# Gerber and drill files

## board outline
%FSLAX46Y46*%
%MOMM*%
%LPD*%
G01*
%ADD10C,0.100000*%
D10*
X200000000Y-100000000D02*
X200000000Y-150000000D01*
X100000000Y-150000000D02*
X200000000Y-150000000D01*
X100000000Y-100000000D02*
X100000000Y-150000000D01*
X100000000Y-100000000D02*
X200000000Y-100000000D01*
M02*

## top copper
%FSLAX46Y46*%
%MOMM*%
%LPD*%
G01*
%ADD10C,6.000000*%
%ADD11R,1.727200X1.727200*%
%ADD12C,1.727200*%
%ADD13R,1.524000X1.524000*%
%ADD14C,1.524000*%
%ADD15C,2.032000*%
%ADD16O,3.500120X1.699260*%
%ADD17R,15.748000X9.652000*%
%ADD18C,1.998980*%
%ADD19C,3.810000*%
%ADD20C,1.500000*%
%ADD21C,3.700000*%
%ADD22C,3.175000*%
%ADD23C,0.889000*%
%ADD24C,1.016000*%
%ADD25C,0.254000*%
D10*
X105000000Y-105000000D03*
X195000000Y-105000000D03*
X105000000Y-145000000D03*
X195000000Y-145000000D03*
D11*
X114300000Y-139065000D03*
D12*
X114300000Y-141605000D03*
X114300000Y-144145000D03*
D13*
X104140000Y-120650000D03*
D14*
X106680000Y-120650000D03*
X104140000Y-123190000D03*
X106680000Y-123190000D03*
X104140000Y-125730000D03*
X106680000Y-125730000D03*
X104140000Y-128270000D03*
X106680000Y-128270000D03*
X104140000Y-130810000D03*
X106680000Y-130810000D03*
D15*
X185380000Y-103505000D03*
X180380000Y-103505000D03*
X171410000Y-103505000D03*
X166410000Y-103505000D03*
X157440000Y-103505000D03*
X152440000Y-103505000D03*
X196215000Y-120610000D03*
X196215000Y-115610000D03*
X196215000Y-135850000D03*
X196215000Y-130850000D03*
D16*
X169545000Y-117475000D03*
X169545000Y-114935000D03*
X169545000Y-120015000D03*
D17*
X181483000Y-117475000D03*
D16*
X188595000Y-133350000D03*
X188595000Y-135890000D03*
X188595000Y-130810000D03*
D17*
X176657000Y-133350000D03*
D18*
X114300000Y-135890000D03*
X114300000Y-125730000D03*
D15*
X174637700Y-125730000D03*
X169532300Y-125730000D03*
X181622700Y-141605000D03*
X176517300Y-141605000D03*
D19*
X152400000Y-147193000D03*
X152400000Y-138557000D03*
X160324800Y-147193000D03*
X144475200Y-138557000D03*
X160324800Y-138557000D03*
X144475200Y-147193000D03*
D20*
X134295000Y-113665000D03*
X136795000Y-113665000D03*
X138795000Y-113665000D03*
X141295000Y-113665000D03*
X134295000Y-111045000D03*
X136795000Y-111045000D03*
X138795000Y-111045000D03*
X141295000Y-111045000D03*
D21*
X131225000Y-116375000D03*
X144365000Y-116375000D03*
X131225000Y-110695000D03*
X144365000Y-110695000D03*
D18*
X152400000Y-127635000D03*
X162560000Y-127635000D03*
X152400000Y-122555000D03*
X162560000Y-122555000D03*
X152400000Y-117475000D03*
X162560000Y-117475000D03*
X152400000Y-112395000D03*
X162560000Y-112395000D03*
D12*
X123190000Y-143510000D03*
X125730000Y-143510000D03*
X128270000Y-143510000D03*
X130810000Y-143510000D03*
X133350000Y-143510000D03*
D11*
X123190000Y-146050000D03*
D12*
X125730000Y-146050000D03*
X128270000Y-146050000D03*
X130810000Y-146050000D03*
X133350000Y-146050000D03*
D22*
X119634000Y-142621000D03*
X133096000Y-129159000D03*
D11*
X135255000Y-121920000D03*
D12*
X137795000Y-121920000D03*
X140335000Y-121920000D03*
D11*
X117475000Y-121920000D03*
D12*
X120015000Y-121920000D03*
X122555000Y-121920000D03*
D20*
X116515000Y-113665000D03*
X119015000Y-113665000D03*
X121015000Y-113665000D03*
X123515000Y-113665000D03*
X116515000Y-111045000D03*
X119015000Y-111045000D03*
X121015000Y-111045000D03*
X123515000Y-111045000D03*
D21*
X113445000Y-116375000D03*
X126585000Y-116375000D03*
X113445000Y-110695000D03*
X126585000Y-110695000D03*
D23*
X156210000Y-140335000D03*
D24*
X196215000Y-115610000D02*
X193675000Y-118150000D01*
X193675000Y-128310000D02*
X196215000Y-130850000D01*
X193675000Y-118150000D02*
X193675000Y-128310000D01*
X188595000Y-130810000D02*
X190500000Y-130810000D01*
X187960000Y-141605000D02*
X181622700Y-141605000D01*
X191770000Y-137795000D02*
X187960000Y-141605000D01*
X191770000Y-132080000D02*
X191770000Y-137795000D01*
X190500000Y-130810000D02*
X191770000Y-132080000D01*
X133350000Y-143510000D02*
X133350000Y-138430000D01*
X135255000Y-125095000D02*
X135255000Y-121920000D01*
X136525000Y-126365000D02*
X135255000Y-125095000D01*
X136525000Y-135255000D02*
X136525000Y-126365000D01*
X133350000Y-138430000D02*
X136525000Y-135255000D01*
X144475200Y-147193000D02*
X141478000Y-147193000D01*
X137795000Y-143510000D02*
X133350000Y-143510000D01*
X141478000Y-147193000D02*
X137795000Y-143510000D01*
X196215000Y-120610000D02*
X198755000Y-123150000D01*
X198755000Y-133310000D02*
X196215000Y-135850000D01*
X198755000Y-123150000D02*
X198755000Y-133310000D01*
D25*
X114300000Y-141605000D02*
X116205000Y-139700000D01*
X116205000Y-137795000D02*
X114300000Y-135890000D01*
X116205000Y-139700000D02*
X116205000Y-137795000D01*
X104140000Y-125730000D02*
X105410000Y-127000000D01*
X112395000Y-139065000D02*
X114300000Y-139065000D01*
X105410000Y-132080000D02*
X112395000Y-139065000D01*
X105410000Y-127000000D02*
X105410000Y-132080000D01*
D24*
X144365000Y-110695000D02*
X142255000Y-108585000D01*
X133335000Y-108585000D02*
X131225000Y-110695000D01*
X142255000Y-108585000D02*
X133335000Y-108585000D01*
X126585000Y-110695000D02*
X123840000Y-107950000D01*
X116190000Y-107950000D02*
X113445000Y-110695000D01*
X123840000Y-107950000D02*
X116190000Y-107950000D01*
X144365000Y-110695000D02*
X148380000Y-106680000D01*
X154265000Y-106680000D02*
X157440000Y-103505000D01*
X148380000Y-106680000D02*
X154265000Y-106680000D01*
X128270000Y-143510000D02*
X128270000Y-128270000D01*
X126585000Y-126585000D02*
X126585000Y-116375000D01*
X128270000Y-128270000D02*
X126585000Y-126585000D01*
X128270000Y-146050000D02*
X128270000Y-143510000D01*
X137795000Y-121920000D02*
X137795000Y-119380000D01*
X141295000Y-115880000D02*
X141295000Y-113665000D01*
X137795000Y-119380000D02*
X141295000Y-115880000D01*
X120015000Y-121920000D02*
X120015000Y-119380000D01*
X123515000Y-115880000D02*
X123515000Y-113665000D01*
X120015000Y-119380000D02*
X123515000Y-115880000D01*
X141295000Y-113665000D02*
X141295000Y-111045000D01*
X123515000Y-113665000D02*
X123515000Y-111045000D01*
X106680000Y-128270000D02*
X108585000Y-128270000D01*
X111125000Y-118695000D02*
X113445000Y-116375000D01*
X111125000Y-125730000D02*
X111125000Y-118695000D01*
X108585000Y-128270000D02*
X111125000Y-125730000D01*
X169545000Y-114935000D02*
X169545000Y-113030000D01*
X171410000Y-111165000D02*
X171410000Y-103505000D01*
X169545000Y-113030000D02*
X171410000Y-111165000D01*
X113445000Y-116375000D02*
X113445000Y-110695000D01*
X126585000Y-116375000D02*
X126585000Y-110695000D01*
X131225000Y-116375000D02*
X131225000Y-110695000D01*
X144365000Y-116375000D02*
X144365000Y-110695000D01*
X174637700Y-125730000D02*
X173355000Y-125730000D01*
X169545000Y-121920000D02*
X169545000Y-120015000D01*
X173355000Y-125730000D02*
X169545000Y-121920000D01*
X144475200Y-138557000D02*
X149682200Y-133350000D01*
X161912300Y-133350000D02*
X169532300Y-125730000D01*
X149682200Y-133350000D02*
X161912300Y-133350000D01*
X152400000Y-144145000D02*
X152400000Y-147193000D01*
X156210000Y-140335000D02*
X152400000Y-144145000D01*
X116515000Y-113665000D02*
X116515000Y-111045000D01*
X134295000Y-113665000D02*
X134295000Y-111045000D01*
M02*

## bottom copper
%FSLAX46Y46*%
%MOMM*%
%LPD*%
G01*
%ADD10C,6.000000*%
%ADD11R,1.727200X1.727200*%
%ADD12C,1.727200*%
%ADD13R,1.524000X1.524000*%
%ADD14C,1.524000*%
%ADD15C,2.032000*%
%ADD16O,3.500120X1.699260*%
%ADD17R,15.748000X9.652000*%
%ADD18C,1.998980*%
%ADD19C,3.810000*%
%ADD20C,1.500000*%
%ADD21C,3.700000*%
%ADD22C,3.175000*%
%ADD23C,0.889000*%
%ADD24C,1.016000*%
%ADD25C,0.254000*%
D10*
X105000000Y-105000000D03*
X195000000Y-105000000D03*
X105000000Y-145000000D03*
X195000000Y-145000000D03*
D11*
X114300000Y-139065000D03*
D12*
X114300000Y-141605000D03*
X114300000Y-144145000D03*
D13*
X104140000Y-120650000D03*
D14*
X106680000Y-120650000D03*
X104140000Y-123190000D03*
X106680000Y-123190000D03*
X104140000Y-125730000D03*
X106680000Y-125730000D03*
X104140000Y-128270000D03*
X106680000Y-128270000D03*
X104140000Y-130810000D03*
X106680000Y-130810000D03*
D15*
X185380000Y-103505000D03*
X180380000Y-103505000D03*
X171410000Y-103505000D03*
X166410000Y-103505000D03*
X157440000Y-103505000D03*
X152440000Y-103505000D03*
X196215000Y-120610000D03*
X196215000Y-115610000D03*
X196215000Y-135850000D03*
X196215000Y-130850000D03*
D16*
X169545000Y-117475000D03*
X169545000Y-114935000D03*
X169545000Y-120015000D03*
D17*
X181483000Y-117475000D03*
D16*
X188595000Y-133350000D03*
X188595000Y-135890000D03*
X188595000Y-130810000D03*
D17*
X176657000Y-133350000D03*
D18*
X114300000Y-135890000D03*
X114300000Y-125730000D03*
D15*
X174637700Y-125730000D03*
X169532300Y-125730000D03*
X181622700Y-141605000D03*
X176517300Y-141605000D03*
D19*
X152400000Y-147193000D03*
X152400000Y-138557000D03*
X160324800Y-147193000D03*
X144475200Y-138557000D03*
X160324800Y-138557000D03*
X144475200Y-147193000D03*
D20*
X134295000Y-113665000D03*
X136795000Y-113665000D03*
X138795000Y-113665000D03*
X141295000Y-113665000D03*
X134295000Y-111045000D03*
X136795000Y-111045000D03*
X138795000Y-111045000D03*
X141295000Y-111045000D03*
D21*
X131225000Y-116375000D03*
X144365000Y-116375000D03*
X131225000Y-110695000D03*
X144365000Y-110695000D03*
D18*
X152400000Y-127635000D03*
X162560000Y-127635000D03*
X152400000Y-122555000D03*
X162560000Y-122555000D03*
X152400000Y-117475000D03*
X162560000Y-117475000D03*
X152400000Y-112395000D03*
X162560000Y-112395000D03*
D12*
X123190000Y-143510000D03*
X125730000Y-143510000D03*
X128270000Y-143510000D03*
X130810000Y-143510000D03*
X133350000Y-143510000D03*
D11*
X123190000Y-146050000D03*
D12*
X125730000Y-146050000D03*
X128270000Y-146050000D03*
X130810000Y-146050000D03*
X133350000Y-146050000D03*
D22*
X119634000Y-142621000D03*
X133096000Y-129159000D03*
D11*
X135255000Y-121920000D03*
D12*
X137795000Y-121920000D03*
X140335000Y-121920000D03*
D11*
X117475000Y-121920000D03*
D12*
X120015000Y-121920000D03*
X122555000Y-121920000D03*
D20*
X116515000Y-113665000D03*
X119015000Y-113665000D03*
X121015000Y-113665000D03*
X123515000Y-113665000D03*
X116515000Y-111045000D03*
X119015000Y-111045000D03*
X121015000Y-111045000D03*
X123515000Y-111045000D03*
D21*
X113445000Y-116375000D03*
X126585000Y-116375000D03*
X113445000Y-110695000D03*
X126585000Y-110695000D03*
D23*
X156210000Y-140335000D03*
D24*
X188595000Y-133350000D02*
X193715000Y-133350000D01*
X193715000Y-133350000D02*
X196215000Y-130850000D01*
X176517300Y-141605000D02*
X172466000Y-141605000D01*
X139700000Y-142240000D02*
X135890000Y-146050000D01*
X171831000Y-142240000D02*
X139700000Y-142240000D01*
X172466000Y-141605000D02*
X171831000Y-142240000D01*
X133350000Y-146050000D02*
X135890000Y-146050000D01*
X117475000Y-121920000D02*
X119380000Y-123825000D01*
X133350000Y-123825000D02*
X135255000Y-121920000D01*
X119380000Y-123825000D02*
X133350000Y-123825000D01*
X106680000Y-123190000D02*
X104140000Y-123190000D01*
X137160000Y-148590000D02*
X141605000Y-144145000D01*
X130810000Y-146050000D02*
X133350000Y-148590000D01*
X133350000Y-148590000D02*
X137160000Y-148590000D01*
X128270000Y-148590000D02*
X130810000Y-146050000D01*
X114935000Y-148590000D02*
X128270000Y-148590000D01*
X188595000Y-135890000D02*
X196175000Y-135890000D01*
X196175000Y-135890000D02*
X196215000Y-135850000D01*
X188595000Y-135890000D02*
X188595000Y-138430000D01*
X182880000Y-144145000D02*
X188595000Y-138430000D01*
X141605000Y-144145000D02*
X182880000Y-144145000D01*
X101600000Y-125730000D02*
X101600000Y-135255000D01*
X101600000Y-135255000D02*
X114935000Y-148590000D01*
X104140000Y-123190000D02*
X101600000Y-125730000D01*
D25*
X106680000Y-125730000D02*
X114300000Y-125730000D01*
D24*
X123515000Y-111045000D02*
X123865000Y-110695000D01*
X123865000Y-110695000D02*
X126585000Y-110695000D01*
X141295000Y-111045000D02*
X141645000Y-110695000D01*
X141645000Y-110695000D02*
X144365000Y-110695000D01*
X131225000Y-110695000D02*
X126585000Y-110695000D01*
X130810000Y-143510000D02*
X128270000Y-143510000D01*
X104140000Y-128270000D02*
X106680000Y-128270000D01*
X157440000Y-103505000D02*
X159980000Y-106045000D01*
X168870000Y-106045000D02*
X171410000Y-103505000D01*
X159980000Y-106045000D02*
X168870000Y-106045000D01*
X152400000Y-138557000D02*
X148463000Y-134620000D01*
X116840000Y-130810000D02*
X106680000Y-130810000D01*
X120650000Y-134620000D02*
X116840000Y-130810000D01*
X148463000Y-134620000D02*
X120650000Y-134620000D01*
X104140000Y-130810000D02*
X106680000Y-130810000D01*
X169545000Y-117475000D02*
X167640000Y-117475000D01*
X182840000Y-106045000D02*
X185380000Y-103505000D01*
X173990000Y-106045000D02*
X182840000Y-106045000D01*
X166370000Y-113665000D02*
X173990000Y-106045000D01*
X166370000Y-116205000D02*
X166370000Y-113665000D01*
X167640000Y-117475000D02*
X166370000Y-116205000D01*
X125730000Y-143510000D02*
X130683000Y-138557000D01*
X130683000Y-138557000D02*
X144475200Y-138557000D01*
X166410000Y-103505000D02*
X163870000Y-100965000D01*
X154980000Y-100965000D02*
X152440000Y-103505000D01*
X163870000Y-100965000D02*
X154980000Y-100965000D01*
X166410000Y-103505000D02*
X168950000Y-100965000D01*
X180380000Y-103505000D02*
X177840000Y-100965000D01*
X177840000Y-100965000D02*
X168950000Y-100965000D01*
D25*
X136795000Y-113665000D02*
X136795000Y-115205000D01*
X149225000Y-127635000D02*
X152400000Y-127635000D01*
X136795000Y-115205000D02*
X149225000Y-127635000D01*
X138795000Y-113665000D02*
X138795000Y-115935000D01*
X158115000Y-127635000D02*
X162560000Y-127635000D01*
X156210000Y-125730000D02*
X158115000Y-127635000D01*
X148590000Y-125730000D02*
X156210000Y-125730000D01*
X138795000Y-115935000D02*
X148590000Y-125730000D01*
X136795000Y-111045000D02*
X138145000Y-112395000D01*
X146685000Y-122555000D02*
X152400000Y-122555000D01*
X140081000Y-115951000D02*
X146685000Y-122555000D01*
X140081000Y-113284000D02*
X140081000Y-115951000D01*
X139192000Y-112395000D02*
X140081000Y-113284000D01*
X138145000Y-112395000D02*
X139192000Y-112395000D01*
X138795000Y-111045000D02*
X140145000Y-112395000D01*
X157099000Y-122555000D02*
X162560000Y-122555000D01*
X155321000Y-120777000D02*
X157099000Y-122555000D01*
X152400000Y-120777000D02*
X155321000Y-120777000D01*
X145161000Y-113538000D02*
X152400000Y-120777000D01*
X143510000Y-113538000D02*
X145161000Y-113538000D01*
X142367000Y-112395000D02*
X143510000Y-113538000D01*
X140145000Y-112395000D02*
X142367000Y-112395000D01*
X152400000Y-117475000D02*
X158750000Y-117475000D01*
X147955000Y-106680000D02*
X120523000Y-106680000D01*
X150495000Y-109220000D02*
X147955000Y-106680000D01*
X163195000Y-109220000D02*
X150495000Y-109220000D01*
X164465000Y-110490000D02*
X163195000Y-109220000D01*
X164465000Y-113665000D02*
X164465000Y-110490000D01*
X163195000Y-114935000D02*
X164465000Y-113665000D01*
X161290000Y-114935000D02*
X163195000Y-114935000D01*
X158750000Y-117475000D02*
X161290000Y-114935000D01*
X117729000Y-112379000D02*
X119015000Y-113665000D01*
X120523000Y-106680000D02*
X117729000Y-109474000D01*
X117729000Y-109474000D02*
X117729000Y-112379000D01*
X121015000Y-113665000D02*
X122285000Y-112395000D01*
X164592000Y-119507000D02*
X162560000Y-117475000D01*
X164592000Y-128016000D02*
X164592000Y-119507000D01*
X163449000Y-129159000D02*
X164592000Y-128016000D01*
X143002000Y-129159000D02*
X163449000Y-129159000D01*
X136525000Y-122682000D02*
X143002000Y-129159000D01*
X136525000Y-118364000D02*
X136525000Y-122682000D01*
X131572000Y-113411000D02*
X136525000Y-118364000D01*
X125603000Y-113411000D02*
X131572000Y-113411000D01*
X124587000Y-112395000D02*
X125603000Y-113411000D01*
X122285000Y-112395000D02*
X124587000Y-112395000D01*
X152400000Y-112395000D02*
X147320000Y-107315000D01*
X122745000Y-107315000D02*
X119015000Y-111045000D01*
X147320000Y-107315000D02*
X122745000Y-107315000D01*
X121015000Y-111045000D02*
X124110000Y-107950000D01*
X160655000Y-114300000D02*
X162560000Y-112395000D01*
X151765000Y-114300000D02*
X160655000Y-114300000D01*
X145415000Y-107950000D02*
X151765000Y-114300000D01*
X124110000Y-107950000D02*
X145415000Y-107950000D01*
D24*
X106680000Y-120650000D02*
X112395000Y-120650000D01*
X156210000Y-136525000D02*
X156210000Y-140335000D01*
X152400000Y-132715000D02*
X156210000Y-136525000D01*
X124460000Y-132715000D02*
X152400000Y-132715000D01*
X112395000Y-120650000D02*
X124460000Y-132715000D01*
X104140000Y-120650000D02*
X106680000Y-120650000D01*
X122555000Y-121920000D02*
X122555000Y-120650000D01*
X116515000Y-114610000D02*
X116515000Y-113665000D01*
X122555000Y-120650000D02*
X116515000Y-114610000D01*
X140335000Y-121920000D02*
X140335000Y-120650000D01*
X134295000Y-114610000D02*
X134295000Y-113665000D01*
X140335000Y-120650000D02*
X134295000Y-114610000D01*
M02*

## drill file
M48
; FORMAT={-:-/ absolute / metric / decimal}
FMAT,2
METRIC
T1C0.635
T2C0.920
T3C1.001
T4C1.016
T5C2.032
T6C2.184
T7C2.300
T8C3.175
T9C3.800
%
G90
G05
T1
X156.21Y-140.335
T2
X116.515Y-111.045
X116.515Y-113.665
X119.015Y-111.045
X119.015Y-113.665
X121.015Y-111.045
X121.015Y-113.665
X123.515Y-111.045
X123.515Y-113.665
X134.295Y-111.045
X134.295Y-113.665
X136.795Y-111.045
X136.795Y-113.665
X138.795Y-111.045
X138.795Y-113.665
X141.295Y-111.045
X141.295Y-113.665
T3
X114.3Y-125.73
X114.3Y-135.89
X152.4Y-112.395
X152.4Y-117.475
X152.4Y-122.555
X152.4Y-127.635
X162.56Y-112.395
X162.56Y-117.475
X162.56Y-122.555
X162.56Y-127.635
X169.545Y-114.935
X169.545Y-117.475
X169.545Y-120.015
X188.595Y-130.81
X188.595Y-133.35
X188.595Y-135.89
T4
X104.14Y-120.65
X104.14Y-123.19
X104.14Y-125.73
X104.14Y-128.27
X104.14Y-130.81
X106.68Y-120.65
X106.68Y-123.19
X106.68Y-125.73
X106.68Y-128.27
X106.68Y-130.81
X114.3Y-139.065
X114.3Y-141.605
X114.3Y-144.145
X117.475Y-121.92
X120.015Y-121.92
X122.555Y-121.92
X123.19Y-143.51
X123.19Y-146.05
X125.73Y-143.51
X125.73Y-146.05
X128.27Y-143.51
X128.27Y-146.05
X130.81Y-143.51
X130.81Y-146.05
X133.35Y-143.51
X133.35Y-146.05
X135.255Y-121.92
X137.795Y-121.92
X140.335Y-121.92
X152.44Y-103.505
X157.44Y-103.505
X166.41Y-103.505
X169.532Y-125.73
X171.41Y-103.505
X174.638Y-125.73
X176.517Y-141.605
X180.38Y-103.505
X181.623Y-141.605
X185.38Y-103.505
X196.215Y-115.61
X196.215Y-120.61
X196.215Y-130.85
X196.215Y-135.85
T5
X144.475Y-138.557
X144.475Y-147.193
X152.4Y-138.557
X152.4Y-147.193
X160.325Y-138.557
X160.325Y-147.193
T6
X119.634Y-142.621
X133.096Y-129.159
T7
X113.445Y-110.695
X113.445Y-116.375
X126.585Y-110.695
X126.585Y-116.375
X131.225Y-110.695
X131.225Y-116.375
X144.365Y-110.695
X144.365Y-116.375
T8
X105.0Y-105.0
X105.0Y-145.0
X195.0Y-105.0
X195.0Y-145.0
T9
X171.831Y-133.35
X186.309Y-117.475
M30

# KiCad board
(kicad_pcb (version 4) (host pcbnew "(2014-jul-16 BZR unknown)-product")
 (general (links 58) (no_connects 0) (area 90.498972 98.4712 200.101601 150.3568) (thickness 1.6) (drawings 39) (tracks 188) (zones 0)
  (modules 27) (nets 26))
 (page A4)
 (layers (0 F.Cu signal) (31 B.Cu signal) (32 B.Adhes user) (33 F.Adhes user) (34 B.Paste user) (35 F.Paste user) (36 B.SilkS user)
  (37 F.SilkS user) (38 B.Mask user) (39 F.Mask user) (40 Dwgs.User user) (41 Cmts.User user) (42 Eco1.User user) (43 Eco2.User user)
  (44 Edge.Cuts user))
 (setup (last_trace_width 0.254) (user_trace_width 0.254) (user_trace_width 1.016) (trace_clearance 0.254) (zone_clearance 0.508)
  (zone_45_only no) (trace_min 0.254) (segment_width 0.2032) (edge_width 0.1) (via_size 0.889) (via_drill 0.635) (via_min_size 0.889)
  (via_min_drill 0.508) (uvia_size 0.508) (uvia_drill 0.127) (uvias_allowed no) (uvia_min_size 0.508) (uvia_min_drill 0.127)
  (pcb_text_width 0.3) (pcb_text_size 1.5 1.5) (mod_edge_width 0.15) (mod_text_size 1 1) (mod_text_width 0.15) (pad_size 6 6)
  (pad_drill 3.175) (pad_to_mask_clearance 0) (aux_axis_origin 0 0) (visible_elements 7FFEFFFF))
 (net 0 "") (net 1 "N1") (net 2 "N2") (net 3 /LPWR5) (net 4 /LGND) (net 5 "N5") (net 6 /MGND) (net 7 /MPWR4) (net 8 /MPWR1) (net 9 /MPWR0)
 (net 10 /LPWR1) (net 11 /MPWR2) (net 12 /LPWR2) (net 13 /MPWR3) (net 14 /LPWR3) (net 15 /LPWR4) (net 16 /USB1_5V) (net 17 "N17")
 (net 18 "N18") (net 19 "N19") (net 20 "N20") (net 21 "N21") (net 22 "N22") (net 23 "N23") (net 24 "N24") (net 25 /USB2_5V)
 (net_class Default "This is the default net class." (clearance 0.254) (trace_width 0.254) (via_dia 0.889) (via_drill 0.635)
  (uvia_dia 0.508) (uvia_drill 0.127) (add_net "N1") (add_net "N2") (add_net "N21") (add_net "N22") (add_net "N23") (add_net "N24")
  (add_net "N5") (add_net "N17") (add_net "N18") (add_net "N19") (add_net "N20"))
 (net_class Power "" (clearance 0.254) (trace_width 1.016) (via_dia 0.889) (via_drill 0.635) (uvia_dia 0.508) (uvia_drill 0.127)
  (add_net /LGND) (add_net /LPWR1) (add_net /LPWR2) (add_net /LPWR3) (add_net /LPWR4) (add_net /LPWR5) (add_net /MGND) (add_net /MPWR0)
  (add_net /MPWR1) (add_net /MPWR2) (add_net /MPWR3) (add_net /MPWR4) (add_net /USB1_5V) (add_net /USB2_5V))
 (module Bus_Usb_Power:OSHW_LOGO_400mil (layer B.Cu) (at 123.825 131.445 180)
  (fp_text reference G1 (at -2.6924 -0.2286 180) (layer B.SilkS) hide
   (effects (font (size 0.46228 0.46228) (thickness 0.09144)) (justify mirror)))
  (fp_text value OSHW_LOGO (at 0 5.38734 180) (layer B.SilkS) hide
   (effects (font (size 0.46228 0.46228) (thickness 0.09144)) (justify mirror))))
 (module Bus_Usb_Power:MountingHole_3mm (layer F.Cu) (at 105 105)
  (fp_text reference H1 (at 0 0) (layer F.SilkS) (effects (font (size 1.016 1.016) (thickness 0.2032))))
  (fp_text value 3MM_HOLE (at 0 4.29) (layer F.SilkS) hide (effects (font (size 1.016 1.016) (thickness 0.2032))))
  (pad 1 thru_hole circle (at 0 0) (size 6 6) (drill 3.175) (layers *.Cu *.SilkS)))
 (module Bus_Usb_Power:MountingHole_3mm (layer F.Cu) (at 195 105)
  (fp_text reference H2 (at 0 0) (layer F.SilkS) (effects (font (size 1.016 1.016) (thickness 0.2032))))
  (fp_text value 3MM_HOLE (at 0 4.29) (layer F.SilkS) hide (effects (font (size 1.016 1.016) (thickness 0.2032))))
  (pad 1 thru_hole circle (at 0 0) (size 6 6) (drill 3.175) (layers *.Cu *.SilkS)))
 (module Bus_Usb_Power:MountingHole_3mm (layer F.Cu) (at 105 145)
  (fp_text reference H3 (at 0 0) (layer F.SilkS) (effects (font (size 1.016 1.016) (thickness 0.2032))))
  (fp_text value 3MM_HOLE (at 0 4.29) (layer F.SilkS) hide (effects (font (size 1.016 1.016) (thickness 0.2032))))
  (pad 1 thru_hole circle (at 0 0) (size 6 6) (drill 3.175) (layers *.Cu *.SilkS)))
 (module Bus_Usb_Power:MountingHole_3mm (layer F.Cu) (at 195 145)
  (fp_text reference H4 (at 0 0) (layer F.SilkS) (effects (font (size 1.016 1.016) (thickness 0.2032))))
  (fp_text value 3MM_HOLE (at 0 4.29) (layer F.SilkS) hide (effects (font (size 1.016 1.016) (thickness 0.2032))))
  (pad 1 thru_hole circle (at 0 0) (size 6 6) (drill 3.175) (layers *.Cu *.SilkS)))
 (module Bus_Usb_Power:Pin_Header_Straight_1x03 (layer F.Cu) (at 114.3 141.605 270)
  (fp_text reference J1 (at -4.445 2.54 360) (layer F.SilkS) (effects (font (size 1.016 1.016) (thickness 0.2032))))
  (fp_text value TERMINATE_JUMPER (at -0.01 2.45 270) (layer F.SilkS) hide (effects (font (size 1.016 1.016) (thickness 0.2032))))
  (pad 1 thru_hole rect (at -2.54 0 270) (size 1.7272 1.7272) (drill 1.016) (layers *.Cu *.Mask F.SilkS) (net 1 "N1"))
  (pad 2 thru_hole circle (at 0 0 270) (size 1.7272 1.7272) (drill 1.016) (layers *.Cu *.Mask F.SilkS) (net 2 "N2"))
  (pad 3 thru_hole circle (at 2.54 0 270) (size 1.7272 1.7272) (drill 1.016) (layers *.Cu *.Mask F.SilkS)))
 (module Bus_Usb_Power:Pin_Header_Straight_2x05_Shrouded (layer F.Cu) (at 105.41 125.73 270)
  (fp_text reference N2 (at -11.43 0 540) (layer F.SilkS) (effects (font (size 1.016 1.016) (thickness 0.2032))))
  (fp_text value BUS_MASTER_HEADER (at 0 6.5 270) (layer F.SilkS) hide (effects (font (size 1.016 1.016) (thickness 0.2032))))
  (pad 1 thru_hole rect (at -5.08 1.27 270) (size 1.524 1.524) (drill 1.016) (layers *.Cu *.Mask F.SilkS) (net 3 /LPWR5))
  (pad 2 thru_hole circle (at -5.08 -1.27 270) (size 1.524 1.524) (drill 1.016) (layers *.Cu *.Mask F.SilkS) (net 3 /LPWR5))
  (pad 3 thru_hole circle (at -2.54 1.27 270) (size 1.524 1.524) (drill 1.016) (layers *.Cu *.Mask F.SilkS) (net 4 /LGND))
  (pad 4 thru_hole circle (at -2.54 -1.27 270) (size 1.524 1.524) (drill 1.016) (layers *.Cu *.Mask F.SilkS) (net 4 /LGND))
  (pad 5 thru_hole circle (at 0 1.27 270) (size 1.524 1.524) (drill 1.016) (layers *.Cu *.Mask F.SilkS) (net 1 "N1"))
  (pad 6 thru_hole circle (at 0 -1.27 270) (size 1.524 1.524) (drill 1.016) (layers *.Cu *.Mask F.SilkS) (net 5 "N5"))
  (pad 7 thru_hole circle (at 2.54 1.27 270) (size 1.524 1.524) (drill 1.016) (layers *.Cu *.Mask F.SilkS) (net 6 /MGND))
  (pad 8 thru_hole circle (at 2.54 -1.27 270) (size 1.524 1.524) (drill 1.016) (layers *.Cu *.Mask F.SilkS) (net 6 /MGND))
  (pad 9 thru_hole circle (at 5.08 1.27 270) (size 1.524 1.524) (drill 1.016) (layers *.Cu *.Mask F.SilkS) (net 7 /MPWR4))
  (pad 10 thru_hole circle (at 5.08 -1.27 270) (size 1.524 1.524) (drill 1.016) (layers *.Cu *.Mask F.SilkS) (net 7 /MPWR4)))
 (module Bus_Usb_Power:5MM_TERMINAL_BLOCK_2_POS (layer F.Cu) (at 182.88 103.505 180)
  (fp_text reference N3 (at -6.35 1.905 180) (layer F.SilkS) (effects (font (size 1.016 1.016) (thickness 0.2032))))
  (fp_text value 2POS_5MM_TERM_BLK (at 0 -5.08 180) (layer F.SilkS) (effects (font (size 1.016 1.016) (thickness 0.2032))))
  (pad 1 thru_hole circle (at -2.5 0 180) (size 2.032 2.032) (drill 1.016) (layers *.Cu *.Mask) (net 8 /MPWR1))
  (pad 2 thru_hole circle (at 2.5 0 180) (size 2.032 2.032) (drill 1.016) (layers *.Cu *.Mask) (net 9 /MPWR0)))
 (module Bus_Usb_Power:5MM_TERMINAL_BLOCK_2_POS (layer F.Cu) (at 168.91 103.505 180)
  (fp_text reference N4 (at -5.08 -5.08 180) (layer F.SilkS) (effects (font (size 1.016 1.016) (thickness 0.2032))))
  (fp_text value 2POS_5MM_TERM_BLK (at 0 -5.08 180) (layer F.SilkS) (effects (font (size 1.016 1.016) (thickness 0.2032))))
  (pad 1 thru_hole circle (at -2.5 0 180) (size 2.032 2.032) (drill 1.016) (layers *.Cu *.Mask) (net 6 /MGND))
  (pad 2 thru_hole circle (at 2.5 0 180) (size 2.032 2.032) (drill 1.016) (layers *.Cu *.Mask) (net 9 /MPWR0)))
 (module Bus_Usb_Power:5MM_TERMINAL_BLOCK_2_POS (layer F.Cu) (at 154.94 103.505 180)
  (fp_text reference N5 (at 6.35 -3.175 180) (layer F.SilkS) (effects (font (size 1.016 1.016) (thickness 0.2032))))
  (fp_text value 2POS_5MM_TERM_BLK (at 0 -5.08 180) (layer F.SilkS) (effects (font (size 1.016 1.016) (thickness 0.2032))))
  (pad 1 thru_hole circle (at -2.5 0 180) (size 2.032 2.032) (drill 1.016) (layers *.Cu *.Mask) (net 6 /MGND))
  (pad 2 thru_hole circle (at 2.5 0 180) (size 2.032 2.032) (drill 1.016) (layers *.Cu *.Mask) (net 9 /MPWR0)))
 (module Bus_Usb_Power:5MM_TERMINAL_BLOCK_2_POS (layer F.Cu) (at 196.215 118.11 90)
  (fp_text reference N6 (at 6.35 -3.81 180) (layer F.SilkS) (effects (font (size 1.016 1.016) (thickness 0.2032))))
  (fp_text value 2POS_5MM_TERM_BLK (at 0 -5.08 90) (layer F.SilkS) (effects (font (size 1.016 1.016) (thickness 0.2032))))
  (pad 1 thru_hole circle (at -2.5 0 90) (size 2.032 2.032) (drill 1.016) (layers *.Cu *.Mask) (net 4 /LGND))
  (pad 2 thru_hole circle (at 2.5 0 90) (size 2.032 2.032) (drill 1.016) (layers *.Cu *.Mask) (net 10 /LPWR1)))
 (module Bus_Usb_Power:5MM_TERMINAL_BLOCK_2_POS (layer F.Cu) (at 196.215 133.35 90)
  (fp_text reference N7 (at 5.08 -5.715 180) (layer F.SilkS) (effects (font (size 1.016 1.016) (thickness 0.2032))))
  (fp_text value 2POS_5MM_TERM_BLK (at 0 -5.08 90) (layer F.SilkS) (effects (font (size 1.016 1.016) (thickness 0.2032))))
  (pad 1 thru_hole circle (at -2.5 0 90) (size 2.032 2.032) (drill 1.016) (layers *.Cu *.Mask) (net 4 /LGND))
  (pad 2 thru_hole circle (at 2.5 0 90) (size 2.032 2.032) (drill 1.016) (layers *.Cu *.Mask) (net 10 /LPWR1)))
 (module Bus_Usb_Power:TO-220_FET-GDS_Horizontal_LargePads (layer F.Cu) (at 169.545 117.475 270)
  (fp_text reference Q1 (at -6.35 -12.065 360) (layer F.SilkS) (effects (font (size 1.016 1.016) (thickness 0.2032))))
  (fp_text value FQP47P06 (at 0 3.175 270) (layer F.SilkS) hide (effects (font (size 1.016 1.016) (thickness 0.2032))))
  (pad D thru_hole oval (at 0 0) (size 3.50012 1.69926) (drill 1.00076) (layers *.Cu *.Mask F.SilkS) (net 8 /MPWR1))
  (pad G thru_hole oval (at -2.54 0) (size 3.50012 1.69926) (drill 1.00076) (layers *.Cu *.Mask F.SilkS) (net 6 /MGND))
  (pad S thru_hole oval (at 2.54 0) (size 3.50012 1.69926) (drill 1.00076) (layers *.Cu *.Mask F.SilkS) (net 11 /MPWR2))
  (pad 2 thru_hole rect (at 0 -16.764) (size 15.748 9.652) (drill 3.79984 (offset -4.826 0)) (layers *.Cu F.SilkS F.Mask)))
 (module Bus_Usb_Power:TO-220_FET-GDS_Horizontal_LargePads (layer F.Cu) (at 188.595 133.35 90)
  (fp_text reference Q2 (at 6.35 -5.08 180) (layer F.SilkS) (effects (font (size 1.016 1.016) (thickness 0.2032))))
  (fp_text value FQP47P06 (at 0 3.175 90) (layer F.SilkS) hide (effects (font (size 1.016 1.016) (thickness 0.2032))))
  (pad D thru_hole oval (at 0 0 180) (size 3.50012 1.69926) (drill 1.00076) (layers *.Cu *.Mask F.SilkS) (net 10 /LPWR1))
  (pad G thru_hole oval (at -2.54 0 180) (size 3.50012 1.69926) (drill 1.00076) (layers *.Cu *.Mask F.SilkS) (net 4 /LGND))
  (pad S thru_hole oval (at 2.54 0 180) (size 3.50012 1.69926) (drill 1.00076) (layers *.Cu *.Mask F.SilkS) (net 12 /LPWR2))
  (pad 2 thru_hole rect (at 0 -16.764 180) (size 15.748 9.652) (drill 3.79984 (offset -4.826 0)) (layers *.Cu F.SilkS F.Mask)))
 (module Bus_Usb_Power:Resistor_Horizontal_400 (layer F.Cu) (at 114.3 130.81 90)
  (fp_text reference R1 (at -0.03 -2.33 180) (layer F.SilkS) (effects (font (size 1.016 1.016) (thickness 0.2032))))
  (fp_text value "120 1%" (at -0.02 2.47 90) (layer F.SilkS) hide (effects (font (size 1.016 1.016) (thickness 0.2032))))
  (pad 1 thru_hole circle (at -5.08 0 90) (size 1.99898 1.99898) (drill 1.00076) (layers *.Cu *.SilkS *.Mask) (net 2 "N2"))
  (pad 2 thru_hole circle (at 5.08 0 90) (size 1.99898 1.99898) (drill 1.00076) (layers *.Cu *.SilkS *.Mask) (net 5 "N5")))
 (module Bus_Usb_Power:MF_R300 (layer F.Cu) (at 172.085 125.73 180)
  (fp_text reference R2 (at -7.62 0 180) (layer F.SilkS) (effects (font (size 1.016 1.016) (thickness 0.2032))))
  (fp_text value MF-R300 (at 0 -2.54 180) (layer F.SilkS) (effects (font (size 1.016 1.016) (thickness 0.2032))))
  (pad 1 thru_hole circle (at -2.5527 0 180) (size 2.032 2.032) (drill 1.016) (layers *.Cu *.Mask) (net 11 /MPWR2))
  (pad 2 thru_hole circle (at 2.5527 0 180) (size 2.032 2.032) (drill 1.016) (layers *.Cu *.Mask) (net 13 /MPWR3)))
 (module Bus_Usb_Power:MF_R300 (layer F.Cu) (at 179.07 141.605 180)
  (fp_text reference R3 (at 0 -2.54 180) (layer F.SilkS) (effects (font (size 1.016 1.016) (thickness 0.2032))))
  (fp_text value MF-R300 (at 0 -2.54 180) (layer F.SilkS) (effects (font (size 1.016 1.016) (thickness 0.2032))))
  (pad 1 thru_hole circle (at -2.5527 0 180) (size 2.032 2.032) (drill 1.016) (layers *.Cu *.Mask) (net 12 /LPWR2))
  (pad 2 thru_hole circle (at 2.5527 0 180) (size 2.032 2.032) (drill 1.016) (layers *.Cu *.Mask) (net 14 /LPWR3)))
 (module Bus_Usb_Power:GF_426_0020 (layer F.Cu) (at 152.4 142.875)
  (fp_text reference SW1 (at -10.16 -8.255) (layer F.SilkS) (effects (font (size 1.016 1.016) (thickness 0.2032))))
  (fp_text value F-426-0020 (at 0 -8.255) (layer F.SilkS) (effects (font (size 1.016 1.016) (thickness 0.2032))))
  (pad 5 thru_hole circle (at 0 4.318) (size 3.81 3.81) (drill 2.032) (layers *.Cu *.Mask) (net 3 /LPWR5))
  (pad 2 thru_hole circle (at 0 -4.318) (size 3.81 3.81) (drill 2.032) (layers *.Cu *.Mask) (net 7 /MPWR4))
  (pad 6 thru_hole circle (at 7.9248 4.318) (size 3.81 3.81) (drill 2.032) (layers *.Cu *.Mask))
  (pad 1 thru_hole circle (at -7.9248 -4.318) (size 3.81 3.81) (drill 2.032) (layers *.Cu *.Mask) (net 13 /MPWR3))
  (pad 3 thru_hole circle (at 7.9248 -4.318) (size 3.81 3.81) (drill 2.032) (layers *.Cu *.Mask))
  (pad 4 thru_hole circle (at -7.9248 4.318) (size 3.81 3.81) (drill 2.032) (layers *.Cu *.Mask) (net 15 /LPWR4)))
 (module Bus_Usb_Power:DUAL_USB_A (layer F.Cu) (at 137.795 113.665)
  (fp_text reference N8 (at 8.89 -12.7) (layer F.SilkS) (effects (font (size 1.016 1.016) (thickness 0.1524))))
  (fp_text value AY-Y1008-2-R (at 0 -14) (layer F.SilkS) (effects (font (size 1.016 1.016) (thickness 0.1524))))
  (pad 1 thru_hole circle (at -3.5 0) (size 1.5 1.5) (drill 0.92) (layers *.Cu *.Mask F.SilkS) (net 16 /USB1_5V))
  (pad 2 thru_hole circle (at -1 0) (size 1.5 1.5) (drill 0.92) (layers *.Cu *.Mask F.SilkS) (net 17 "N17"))
  (pad 3 thru_hole circle (at 1 0) (size 1.5 1.5) (drill 0.92) (layers *.Cu *.Mask F.SilkS) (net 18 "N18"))
  (pad 4 thru_hole circle (at 3.5 0) (size 1.5 1.5) (drill 0.92) (layers *.Cu *.Mask F.SilkS) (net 6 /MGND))
  (pad 5 thru_hole circle (at -3.5 -2.62) (size 1.5 1.5) (drill 0.92) (layers *.Cu *.Mask F.SilkS) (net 16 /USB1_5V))
  (pad 6 thru_hole circle (at -1 -2.62) (size 1.5 1.5) (drill 0.92) (layers *.Cu *.Mask F.SilkS) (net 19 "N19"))
  (pad 7 thru_hole circle (at 1 -2.62) (size 1.5 1.5) (drill 0.92) (layers *.Cu *.Mask F.SilkS) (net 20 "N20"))
  (pad 8 thru_hole circle (at 3.5 -2.62) (size 1.5 1.5) (drill 0.92) (layers *.Cu *.Mask F.SilkS) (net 6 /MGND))
  (pad 9 thru_hole circle (at -6.57 2.71) (size 3.7 3.7) (drill 2.3) (layers *.Cu *.Mask F.SilkS) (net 6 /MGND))
  (pad 10 thru_hole circle (at 6.57 2.71) (size 3.7 3.7) (drill 2.3) (layers *.Cu *.Mask F.SilkS) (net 6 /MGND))
  (pad 11 thru_hole circle (at -6.57 -2.97) (size 3.7 3.7) (drill 2.3) (layers *.Cu *.Mask F.SilkS) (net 6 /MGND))
  (pad 12 thru_hole circle (at 6.57 -2.97) (size 3.7 3.7) (drill 2.3) (layers *.Cu *.Mask F.SilkS) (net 6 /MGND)))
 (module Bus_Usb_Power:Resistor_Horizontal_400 (layer F.Cu) (at 157.48 127.635)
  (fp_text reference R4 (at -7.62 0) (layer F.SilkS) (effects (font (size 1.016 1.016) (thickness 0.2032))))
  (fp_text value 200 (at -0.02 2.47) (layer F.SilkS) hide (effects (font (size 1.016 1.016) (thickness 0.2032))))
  (pad 1 thru_hole circle (at -5.08 0) (size 1.99898 1.99898) (drill 1.00076) (layers *.Cu *.SilkS *.Mask) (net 17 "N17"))
  (pad 2 thru_hole circle (at 5.08 0) (size 1.99898 1.99898) (drill 1.00076) (layers *.Cu *.SilkS *.Mask) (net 18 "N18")))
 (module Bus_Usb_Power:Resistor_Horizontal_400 (layer F.Cu) (at 157.48 122.555)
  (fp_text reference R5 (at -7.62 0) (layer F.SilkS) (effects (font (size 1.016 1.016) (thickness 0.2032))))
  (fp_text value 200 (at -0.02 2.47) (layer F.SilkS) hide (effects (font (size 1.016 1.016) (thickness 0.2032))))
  (pad 1 thru_hole circle (at -5.08 0) (size 1.99898 1.99898) (drill 1.00076) (layers *.Cu *.SilkS *.Mask) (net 19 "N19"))
  (pad 2 thru_hole circle (at 5.08 0) (size 1.99898 1.99898) (drill 1.00076) (layers *.Cu *.SilkS *.Mask) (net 20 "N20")))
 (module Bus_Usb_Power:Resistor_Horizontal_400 (layer F.Cu) (at 157.48 117.475)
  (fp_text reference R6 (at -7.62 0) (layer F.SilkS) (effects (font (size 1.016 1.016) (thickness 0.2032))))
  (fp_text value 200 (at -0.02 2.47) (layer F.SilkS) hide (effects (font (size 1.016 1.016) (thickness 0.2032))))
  (pad 1 thru_hole circle (at -5.08 0) (size 1.99898 1.99898) (drill 1.00076) (layers *.Cu *.SilkS *.Mask) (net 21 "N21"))
  (pad 2 thru_hole circle (at 5.08 0) (size 1.99898 1.99898) (drill 1.00076) (layers *.Cu *.SilkS *.Mask) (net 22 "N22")))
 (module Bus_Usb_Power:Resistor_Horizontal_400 (layer F.Cu) (at 157.48 112.395)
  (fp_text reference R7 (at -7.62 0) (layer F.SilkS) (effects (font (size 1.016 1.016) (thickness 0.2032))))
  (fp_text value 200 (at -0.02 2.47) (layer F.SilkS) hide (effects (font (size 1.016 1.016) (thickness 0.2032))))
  (pad 1 thru_hole circle (at -5.08 0) (size 1.99898 1.99898) (drill 1.00076) (layers *.Cu *.SilkS *.Mask) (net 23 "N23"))
  (pad 2 thru_hole circle (at 5.08 0) (size 1.99898 1.99898) (drill 1.00076) (layers *.Cu *.SilkS *.Mask) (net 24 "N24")))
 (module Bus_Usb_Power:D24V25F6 (layer F.Cu) (at 126.365 135.89)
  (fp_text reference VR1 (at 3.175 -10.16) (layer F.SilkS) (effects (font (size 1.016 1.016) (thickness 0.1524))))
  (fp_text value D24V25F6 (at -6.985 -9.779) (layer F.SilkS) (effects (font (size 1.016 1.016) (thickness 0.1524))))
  (pad 2 thru_hole circle (at -3.175 7.62) (size 1.7272 1.7272) (drill 1.016) (layers *.Cu *.Mask F.SilkS))
  (pad 4 thru_hole circle (at -0.635 7.62) (size 1.7272 1.7272) (drill 1.016) (layers *.Cu *.Mask F.SilkS) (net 13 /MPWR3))
  (pad 6 thru_hole circle (at 1.905 7.62) (size 1.7272 1.7272) (drill 1.016) (layers *.Cu *.Mask F.SilkS) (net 6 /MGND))
  (pad 8 thru_hole circle (at 4.445 7.62) (size 1.7272 1.7272) (drill 1.016) (layers *.Cu *.Mask F.SilkS) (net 6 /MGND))
  (pad 10 thru_hole circle (at 6.985 7.62) (size 1.7272 1.7272) (drill 1.016) (layers *.Cu *.Mask F.SilkS) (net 15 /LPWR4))
  (pad 1 thru_hole rect (at -3.175 10.16) (size 1.7272 1.7272) (drill 1.016) (layers *.Cu *.Mask F.SilkS))
  (pad 3 thru_hole circle (at -0.635 10.16) (size 1.7272 1.7272) (drill 1.016) (layers *.Cu *.Mask F.SilkS))
  (pad 5 thru_hole circle (at 1.905 10.16) (size 1.7272 1.7272) (drill 1.016) (layers *.Cu *.Mask F.SilkS) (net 6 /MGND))
  (pad 7 thru_hole circle (at 4.445 10.16) (size 1.7272 1.7272) (drill 1.016) (layers *.Cu *.Mask F.SilkS) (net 4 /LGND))
  (pad 9 thru_hole circle (at 6.985 10.16) (size 1.7272 1.7272) (drill 1.016) (layers *.Cu *.Mask F.SilkS) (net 14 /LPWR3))
  (pad 11 thru_hole circle (at -6.731 6.731) (size 3.175 3.175) (drill 2.1844) (layers *.Cu *.Mask F.SilkS))
  (pad 12 thru_hole circle (at 6.731 -6.731) (size 3.175 3.175) (drill 2.1844) (layers *.Cu *.Mask F.SilkS)))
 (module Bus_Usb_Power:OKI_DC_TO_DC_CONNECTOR (layer F.Cu) (at 137.795 121.92)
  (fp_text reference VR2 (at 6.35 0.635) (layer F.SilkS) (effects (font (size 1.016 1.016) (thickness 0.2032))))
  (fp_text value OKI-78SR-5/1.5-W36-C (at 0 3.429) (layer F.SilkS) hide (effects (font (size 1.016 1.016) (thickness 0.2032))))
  (pad 1 thru_hole rect (at -2.54 0) (size 1.7272 1.7272) (drill 1.016) (layers *.Cu *.Mask F.SilkS) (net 15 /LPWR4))
  (pad 2 thru_hole circle (at 0 0) (size 1.7272 1.7272) (drill 1.016) (layers *.Cu *.Mask F.SilkS) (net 6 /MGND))
  (pad 3 thru_hole circle (at 2.54 0) (size 1.7272 1.7272) (drill 1.016) (layers *.Cu *.Mask F.SilkS) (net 16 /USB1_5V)))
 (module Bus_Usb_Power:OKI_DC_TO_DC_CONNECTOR (layer F.Cu) (at 120.015 121.92)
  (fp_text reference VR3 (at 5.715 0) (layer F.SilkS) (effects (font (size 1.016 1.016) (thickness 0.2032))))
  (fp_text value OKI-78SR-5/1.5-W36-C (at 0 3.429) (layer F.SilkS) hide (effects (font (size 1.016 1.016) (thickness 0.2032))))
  (pad 1 thru_hole rect (at -2.54 0) (size 1.7272 1.7272) (drill 1.016) (layers *.Cu *.Mask F.SilkS) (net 15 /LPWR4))
  (pad 2 thru_hole circle (at 0 0) (size 1.7272 1.7272) (drill 1.016) (layers *.Cu *.Mask F.SilkS) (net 6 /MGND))
  (pad 3 thru_hole circle (at 2.54 0) (size 1.7272 1.7272) (drill 1.016) (layers *.Cu *.Mask F.SilkS) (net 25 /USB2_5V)))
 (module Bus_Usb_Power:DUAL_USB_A (layer F.Cu) (at 120.015 113.665)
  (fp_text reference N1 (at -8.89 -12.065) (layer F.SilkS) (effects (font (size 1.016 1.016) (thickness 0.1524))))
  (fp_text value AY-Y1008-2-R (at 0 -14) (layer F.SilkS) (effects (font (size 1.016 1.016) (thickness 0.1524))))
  (pad 1 thru_hole circle (at -3.5 0) (size 1.5 1.5) (drill 0.92) (layers *.Cu *.Mask F.SilkS) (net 25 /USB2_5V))
  (pad 2 thru_hole circle (at -1 0) (size 1.5 1.5) (drill 0.92) (layers *.Cu *.Mask F.SilkS) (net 21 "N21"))
  (pad 3 thru_hole circle (at 1 0) (size 1.5 1.5) (drill 0.92) (layers *.Cu *.Mask F.SilkS) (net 22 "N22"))
  (pad 4 thru_hole circle (at 3.5 0) (size 1.5 1.5) (drill 0.92) (layers *.Cu *.Mask F.SilkS) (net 6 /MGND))
  (pad 5 thru_hole circle (at -3.5 -2.62) (size 1.5 1.5) (drill 0.92) (layers *.Cu *.Mask F.SilkS) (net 25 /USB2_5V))
  (pad 6 thru_hole circle (at -1 -2.62) (size 1.5 1.5) (drill 0.92) (layers *.Cu *.Mask F.SilkS) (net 23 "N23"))
  (pad 7 thru_hole circle (at 1 -2.62) (size 1.5 1.5) (drill 0.92) (layers *.Cu *.Mask F.SilkS) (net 24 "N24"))
  (pad 8 thru_hole circle (at 3.5 -2.62) (size 1.5 1.5) (drill 0.92) (layers *.Cu *.Mask F.SilkS) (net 6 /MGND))
  (pad 9 thru_hole circle (at -6.57 2.71) (size 3.7 3.7) (drill 2.3) (layers *.Cu *.Mask F.SilkS) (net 6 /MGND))
  (pad 10 thru_hole circle (at 6.57 2.71) (size 3.7 3.7) (drill 2.3) (layers *.Cu *.Mask F.SilkS) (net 6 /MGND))
  (pad 11 thru_hole circle (at -6.57 -2.97) (size 3.7 3.7) (drill 2.3) (layers *.Cu *.Mask F.SilkS) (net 6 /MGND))
  (pad 12 thru_hole circle (at 6.57 -2.97) (size 3.7 3.7) (drill 2.3) (layers *.Cu *.Mask F.SilkS) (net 6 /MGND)))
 (gr_line (start 200 100) (end 200 150) (angle 90) (layer Edge.Cuts) (width 0.1))
 (gr_line (start 100 150) (end 200 150) (angle 90) (layer Edge.Cuts) (width 0.1))
 (gr_line (start 100 100) (end 100 150) (angle 90) (layer Edge.Cuts) (width 0.1))
 (gr_line (start 100 100) (end 200 100) (angle 90) (layer Edge.Cuts) (width 0.1))
 (segment (start 188.595 133.35) (end 193.715 133.35) (width 1.016) (layer B.Cu) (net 10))
 (segment (start 193.715 133.35) (end 196.215 130.85) (width 1.016) (layer B.Cu) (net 10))
 (segment (start 196.215 115.61) (end 193.675 118.15) (width 1.016) (layer F.Cu) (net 10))
 (segment (start 193.675 128.31) (end 196.215 130.85) (width 1.016) (layer F.Cu) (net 10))
 (segment (start 193.675 118.15) (end 193.675 128.31) (width 1.016) (layer F.Cu) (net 10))
 (segment (start 176.5173 141.605) (end 172.466 141.605) (width 1.016) (layer B.Cu) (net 14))
 (segment (start 139.7 142.24) (end 135.89 146.05) (width 1.016) (layer B.Cu) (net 14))
 (segment (start 171.831 142.24) (end 139.7 142.24) (width 1.016) (layer B.Cu) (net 14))
 (segment (start 172.466 141.605) (end 171.831 142.24) (width 1.016) (layer B.Cu) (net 14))
 (segment (start 133.35 146.05) (end 135.89 146.05) (width 1.016) (layer B.Cu) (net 14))
 (segment (start 188.595 130.81) (end 190.5 130.81) (width 1.016) (layer F.Cu) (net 12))
 (segment (start 187.96 141.605) (end 181.6227 141.605) (width 1.016) (layer F.Cu) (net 12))
 (segment (start 191.77 137.795) (end 187.96 141.605) (width 1.016) (layer F.Cu) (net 12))
 (segment (start 191.77 132.08) (end 191.77 137.795) (width 1.016) (layer F.Cu) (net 12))
 (segment (start 190.5 130.81) (end 191.77 132.08) (width 1.016) (layer F.Cu) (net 12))
 (segment (start 117.475 121.92) (end 119.38 123.825) (width 1.016) (layer B.Cu) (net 15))
 (segment (start 133.35 123.825) (end 135.255 121.92) (width 1.016) (layer B.Cu) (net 15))
 (segment (start 119.38 123.825) (end 133.35 123.825) (width 1.016) (layer B.Cu) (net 15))
 (segment (start 133.35 143.51) (end 133.35 138.43) (width 1.016) (layer F.Cu) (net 15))
 (segment (start 135.255 125.095) (end 135.255 121.92) (width 1.016) (layer F.Cu) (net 15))
 (segment (start 136.525 126.365) (end 135.255 125.095) (width 1.016) (layer F.Cu) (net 15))
 (segment (start 136.525 135.255) (end 136.525 126.365) (width 1.016) (layer F.Cu) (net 15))
 (segment (start 133.35 138.43) (end 136.525 135.255) (width 1.016) (layer F.Cu) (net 15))
 (segment (start 144.4752 147.193) (end 141.478 147.193) (width 1.016) (layer F.Cu) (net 15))
 (segment (start 137.795 143.51) (end 133.35 143.51) (width 1.016) (layer F.Cu) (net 15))
 (segment (start 141.478 147.193) (end 137.795 143.51) (width 1.016) (layer F.Cu) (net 15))
 (segment (start 106.68 123.19) (end 104.14 123.19) (width 1.016) (layer B.Cu) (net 4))
 (segment (start 137.16 148.59) (end 141.605 144.145) (width 1.016) (layer B.Cu) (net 4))
 (segment (start 130.81 146.05) (end 133.35 148.59) (width 1.016) (layer B.Cu) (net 4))
 (segment (start 133.35 148.59) (end 137.16 148.59) (width 1.016) (layer B.Cu) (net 4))
 (segment (start 128.27 148.59) (end 130.81 146.05) (width 1.016) (layer B.Cu) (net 4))
 (segment (start 114.935 148.59) (end 128.27 148.59) (width 1.016) (layer B.Cu) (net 4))
 (segment (start 188.595 135.89) (end 196.175 135.89) (width 1.016) (layer B.Cu) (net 4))
 (segment (start 196.175 135.89) (end 196.215 135.85) (width 1.016) (layer B.Cu) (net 4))
 (segment (start 196.215 120.61) (end 198.755 123.15) (width 1.016) (layer F.Cu) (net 4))
 (segment (start 198.755 133.31) (end 196.215 135.85) (width 1.016) (layer F.Cu) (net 4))
 (segment (start 198.755 123.15) (end 198.755 133.31) (width 1.016) (layer F.Cu) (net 4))
 (segment (start 188.595 135.89) (end 188.595 138.43) (width 1.016) (layer B.Cu) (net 4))
 (segment (start 182.88 144.145) (end 188.595 138.43) (width 1.016) (layer B.Cu) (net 4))
 (segment (start 141.605 144.145) (end 182.88 144.145) (width 1.016) (layer B.Cu) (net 4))
 (segment (start 101.6 125.73) (end 101.6 135.255) (width 1.016) (layer B.Cu) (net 4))
 (segment (start 101.6 135.255) (end 114.935 148.59) (width 1.016) (layer B.Cu) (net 4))
 (segment (start 104.14 123.19) (end 101.6 125.73) (width 1.016) (layer B.Cu) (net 4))
 (segment (start 114.3 141.605) (end 116.205 139.7) (width 0.254) (layer F.Cu) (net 2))
 (segment (start 116.205 137.795) (end 114.3 135.89) (width 0.254) (layer F.Cu) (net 2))
 (segment (start 116.205 139.7) (end 116.205 137.795) (width 0.254) (layer F.Cu) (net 2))
 (segment (start 104.14 125.73) (end 105.41 127) (width 0.254) (layer F.Cu) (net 1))
 (segment (start 112.395 139.065) (end 114.3 139.065) (width 0.254) (layer F.Cu) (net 1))
 (segment (start 105.41 132.08) (end 112.395 139.065) (width 0.254) (layer F.Cu) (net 1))
 (segment (start 105.41 127) (end 105.41 132.08) (width 0.254) (layer F.Cu) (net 1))
 (segment (start 106.68 125.73) (end 114.3 125.73) (width 0.254) (layer B.Cu) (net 5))
 (segment (start 123.515 111.045) (end 123.865 110.695) (width 1.016) (layer B.Cu) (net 6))
 (segment (start 123.865 110.695) (end 126.585 110.695) (width 1.016) (layer B.Cu) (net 6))
 (segment (start 141.295 111.045) (end 141.645 110.695) (width 1.016) (layer B.Cu) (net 6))
 (segment (start 141.645 110.695) (end 144.365 110.695) (width 1.016) (layer B.Cu) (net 6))
 (segment (start 144.365 110.695) (end 142.255 108.585) (width 1.016) (layer F.Cu) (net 6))
 (segment (start 133.335 108.585) (end 131.225 110.695) (width 1.016) (layer F.Cu) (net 6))
 (segment (start 142.255 108.585) (end 133.335 108.585) (width 1.016) (layer F.Cu) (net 6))
 (segment (start 126.585 110.695) (end 123.84 107.95) (width 1.016) (layer F.Cu) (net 6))
 (segment (start 116.19 107.95) (end 113.445 110.695) (width 1.016) (layer F.Cu) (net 6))
 (segment (start 123.84 107.95) (end 116.19 107.95) (width 1.016) (layer F.Cu) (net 6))
 (segment (start 131.225 110.695) (end 126.585 110.695) (width 1.016) (layer B.Cu) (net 6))
 (segment (start 144.365 110.695) (end 148.38 106.68) (width 1.016) (layer F.Cu) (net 6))
 (segment (start 154.265 106.68) (end 157.44 103.505) (width 1.016) (layer F.Cu) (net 6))
 (segment (start 148.38 106.68) (end 154.265 106.68) (width 1.016) (layer F.Cu) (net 6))
 (segment (start 128.27 143.51) (end 128.27 128.27) (width 1.016) (layer F.Cu) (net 6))
 (segment (start 126.585 126.585) (end 126.585 116.375) (width 1.016) (layer F.Cu) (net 6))
 (segment (start 128.27 128.27) (end 126.585 126.585) (width 1.016) (layer F.Cu) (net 6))
 (segment (start 130.81 143.51) (end 128.27 143.51) (width 1.016) (layer B.Cu) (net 6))
 (segment (start 128.27 146.05) (end 128.27 143.51) (width 1.016) (layer F.Cu) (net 6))
 (segment (start 137.795 121.92) (end 137.795 119.38) (width 1.016) (layer F.Cu) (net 6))
 (segment (start 141.295 115.88) (end 141.295 113.665) (width 1.016) (layer F.Cu) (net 6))
 (segment (start 137.795 119.38) (end 141.295 115.88) (width 1.016) (layer F.Cu) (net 6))
 (segment (start 120.015 121.92) (end 120.015 119.38) (width 1.016) (layer F.Cu) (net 6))
 (segment (start 123.515 115.88) (end 123.515 113.665) (width 1.016) (layer F.Cu) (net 6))
 (segment (start 120.015 119.38) (end 123.515 115.88) (width 1.016) (layer F.Cu) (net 6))
 (segment (start 141.295 113.665) (end 141.295 111.045) (width 1.016) (layer F.Cu) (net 6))
 (segment (start 123.515 113.665) (end 123.515 111.045) (width 1.016) (layer F.Cu) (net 6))
 (segment (start 106.68 128.27) (end 108.585 128.27) (width 1.016) (layer F.Cu) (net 6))
 (segment (start 111.125 118.695) (end 113.445 116.375) (width 1.016) (layer F.Cu) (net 6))
 (segment (start 111.125 125.73) (end 111.125 118.695) (width 1.016) (layer F.Cu) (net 6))
 (segment (start 108.585 128.27) (end 111.125 125.73) (width 1.016) (layer F.Cu) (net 6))
 (segment (start 104.14 128.27) (end 106.68 128.27) (width 1.016) (layer B.Cu) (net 6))
 (segment (start 169.545 114.935) (end 169.545 113.03) (width 1.016) (layer F.Cu) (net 6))
 (segment (start 171.41 111.165) (end 171.41 103.505) (width 1.016) (layer F.Cu) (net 6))
 (segment (start 169.545 113.03) (end 171.41 111.165) (width 1.016) (layer F.Cu) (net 6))
 (segment (start 113.445 116.375) (end 113.445 110.695) (width 1.016) (layer F.Cu) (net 6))
 (segment (start 126.585 116.375) (end 126.585 110.695) (width 1.016) (layer F.Cu) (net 6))
 (segment (start 131.225 116.375) (end 131.225 110.695) (width 1.016) (layer F.Cu) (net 6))
 (segment (start 144.365 116.375) (end 144.365 110.695) (width 1.016) (layer F.Cu) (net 6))
 (segment (start 157.44 103.505) (end 159.98 106.045) (width 1.016) (layer B.Cu) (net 6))
 (segment (start 168.87 106.045) (end 171.41 103.505) (width 1.016) (layer B.Cu) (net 6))
 (segment (start 159.98 106.045) (end 168.87 106.045) (width 1.016) (layer B.Cu) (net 6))
 (segment (start 152.4 138.557) (end 148.463 134.62) (width 1.016) (layer B.Cu) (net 7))
 (segment (start 116.84 130.81) (end 106.68 130.81) (width 1.016) (layer B.Cu) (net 7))
 (segment (start 120.65 134.62) (end 116.84 130.81) (width 1.016) (layer B.Cu) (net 7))
 (segment (start 148.463 134.62) (end 120.65 134.62) (width 1.016) (layer B.Cu) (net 7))
 (segment (start 104.14 130.81) (end 106.68 130.81) (width 1.016) (layer B.Cu) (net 7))
 (segment (start 169.545 117.475) (end 167.64 117.475) (width 1.016) (layer B.Cu) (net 8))
 (segment (start 182.84 106.045) (end 185.38 103.505) (width 1.016) (layer B.Cu) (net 8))
 (segment (start 173.99 106.045) (end 182.84 106.045) (width 1.016) (layer B.Cu) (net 8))
 (segment (start 166.37 113.665) (end 173.99 106.045) (width 1.016) (layer B.Cu) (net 8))
 (segment (start 166.37 116.205) (end 166.37 113.665) (width 1.016) (layer B.Cu) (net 8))
 (segment (start 167.64 117.475) (end 166.37 116.205) (width 1.016) (layer B.Cu) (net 8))
 (segment (start 174.6377 125.73) (end 173.355 125.73) (width 1.016) (layer F.Cu) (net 11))
 (segment (start 169.545 121.92) (end 169.545 120.015) (width 1.016) (layer F.Cu) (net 11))
 (segment (start 173.355 125.73) (end 169.545 121.92) (width 1.016) (layer F.Cu) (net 11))
 (segment (start 144.4752 138.557) (end 149.6822 133.35) (width 1.016) (layer F.Cu) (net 13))
 (segment (start 161.9123 133.35) (end 169.5323 125.73) (width 1.016) (layer F.Cu) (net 13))
 (segment (start 149.6822 133.35) (end 161.9123 133.35) (width 1.016) (layer F.Cu) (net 13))
 (segment (start 125.73 143.51) (end 130.683 138.557) (width 1.016) (layer B.Cu) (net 13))
 (segment (start 130.683 138.557) (end 144.4752 138.557) (width 1.016) (layer B.Cu) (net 13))
 (segment (start 166.41 103.505) (end 163.87 100.965) (width 1.016) (layer B.Cu) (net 9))
 (segment (start 154.98 100.965) (end 152.44 103.505) (width 1.016) (layer B.Cu) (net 9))
 (segment (start 163.87 100.965) (end 154.98 100.965) (width 1.016) (layer B.Cu) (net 9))
 (segment (start 166.41 103.505) (end 168.95 100.965) (width 1.016) (layer B.Cu) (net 9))
 (segment (start 180.38 103.505) (end 177.84 100.965) (width 1.016) (layer B.Cu) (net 9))
 (segment (start 177.84 100.965) (end 168.95 100.965) (width 1.016) (layer B.Cu) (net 9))
 (segment (start 136.795 113.665) (end 136.795 115.205) (width 0.254) (layer B.Cu) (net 17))
 (segment (start 149.225 127.635) (end 152.4 127.635) (width 0.254) (layer B.Cu) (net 17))
 (segment (start 136.795 115.205) (end 149.225 127.635) (width 0.254) (layer B.Cu) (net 17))
 (segment (start 138.795 113.665) (end 138.795 115.935) (width 0.254) (layer B.Cu) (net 18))
 (segment (start 158.115 127.635) (end 162.56 127.635) (width 0.254) (layer B.Cu) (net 18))
 (segment (start 156.21 125.73) (end 158.115 127.635) (width 0.254) (layer B.Cu) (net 18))
 (segment (start 148.59 125.73) (end 156.21 125.73) (width 0.254) (layer B.Cu) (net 18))
 (segment (start 138.795 115.935) (end 148.59 125.73) (width 0.254) (layer B.Cu) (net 18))
 (segment (start 136.795 111.045) (end 138.145 112.395) (width 0.254) (layer B.Cu) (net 19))
 (segment (start 146.685 122.555) (end 152.4 122.555) (width 0.254) (layer B.Cu) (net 19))
 (segment (start 140.081 115.951) (end 146.685 122.555) (width 0.254) (layer B.Cu) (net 19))
 (segment (start 140.081 113.284) (end 140.081 115.951) (width 0.254) (layer B.Cu) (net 19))
 (segment (start 139.192 112.395) (end 140.081 113.284) (width 0.254) (layer B.Cu) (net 19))
 (segment (start 138.145 112.395) (end 139.192 112.395) (width 0.254) (layer B.Cu) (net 19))
 (segment (start 138.795 111.045) (end 140.145 112.395) (width 0.254) (layer B.Cu) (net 20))
 (segment (start 157.099 122.555) (end 162.56 122.555) (width 0.254) (layer B.Cu) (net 20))
 (segment (start 155.321 120.777) (end 157.099 122.555) (width 0.254) (layer B.Cu) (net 20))
 (segment (start 152.4 120.777) (end 155.321 120.777) (width 0.254) (layer B.Cu) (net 20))
 (segment (start 145.161 113.538) (end 152.4 120.777) (width 0.254) (layer B.Cu) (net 20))
 (segment (start 143.51 113.538) (end 145.161 113.538) (width 0.254) (layer B.Cu) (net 20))
 (segment (start 142.367 112.395) (end 143.51 113.538) (width 0.254) (layer B.Cu) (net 20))
 (segment (start 140.145 112.395) (end 142.367 112.395) (width 0.254) (layer B.Cu) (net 20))
 (segment (start 152.4 117.475) (end 158.75 117.475) (width 0.254) (layer B.Cu) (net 21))
 (segment (start 147.955 106.68) (end 120.523 106.68) (width 0.254) (layer B.Cu) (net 21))
 (segment (start 150.495 109.22) (end 147.955 106.68) (width 0.254) (layer B.Cu) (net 21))
 (segment (start 163.195 109.22) (end 150.495 109.22) (width 0.254) (layer B.Cu) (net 21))
 (segment (start 164.465 110.49) (end 163.195 109.22) (width 0.254) (layer B.Cu) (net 21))
 (segment (start 164.465 113.665) (end 164.465 110.49) (width 0.254) (layer B.Cu) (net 21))
 (segment (start 163.195 114.935) (end 164.465 113.665) (width 0.254) (layer B.Cu) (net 21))
 (segment (start 161.29 114.935) (end 163.195 114.935) (width 0.254) (layer B.Cu) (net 21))
 (segment (start 158.75 117.475) (end 161.29 114.935) (width 0.254) (layer B.Cu) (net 21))
 (segment (start 117.729 112.379) (end 119.015 113.665) (width 0.254) (layer B.Cu) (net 21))
 (segment (start 120.523 106.68) (end 117.729 109.474) (width 0.254) (layer B.Cu) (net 21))
 (segment (start 117.729 109.474) (end 117.729 112.379) (width 0.254) (layer B.Cu) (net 21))
 (segment (start 121.015 113.665) (end 122.285 112.395) (width 0.254) (layer B.Cu) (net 22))
 (segment (start 164.592 119.507) (end 162.56 117.475) (width 0.254) (layer B.Cu) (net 22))
 (segment (start 164.592 128.016) (end 164.592 119.507) (width 0.254) (layer B.Cu) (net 22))
 (segment (start 163.449 129.159) (end 164.592 128.016) (width 0.254) (layer B.Cu) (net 22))
 (segment (start 143.002 129.159) (end 163.449 129.159) (width 0.254) (layer B.Cu) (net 22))
 (segment (start 136.525 122.682) (end 143.002 129.159) (width 0.254) (layer B.Cu) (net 22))
 (segment (start 136.525 118.364) (end 136.525 122.682) (width 0.254) (layer B.Cu) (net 22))
 (segment (start 131.572 113.411) (end 136.525 118.364) (width 0.254) (layer B.Cu) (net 22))
 (segment (start 125.603 113.411) (end 131.572 113.411) (width 0.254) (layer B.Cu) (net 22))
 (segment (start 124.587 112.395) (end 125.603 113.411) (width 0.254) (layer B.Cu) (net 22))
 (segment (start 122.285 112.395) (end 124.587 112.395) (width 0.254) (layer B.Cu) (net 22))
 (segment (start 152.4 112.395) (end 147.32 107.315) (width 0.254) (layer B.Cu) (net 23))
 (segment (start 122.745 107.315) (end 119.015 111.045) (width 0.254) (layer B.Cu) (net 23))
 (segment (start 147.32 107.315) (end 122.745 107.315) (width 0.254) (layer B.Cu) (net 23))
 (segment (start 121.015 111.045) (end 124.11 107.95) (width 0.254) (layer B.Cu) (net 24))
 (segment (start 160.655 114.3) (end 162.56 112.395) (width 0.254) (layer B.Cu) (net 24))
 (segment (start 151.765 114.3) (end 160.655 114.3) (width 0.254) (layer B.Cu) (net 24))
 (segment (start 145.415 107.95) (end 151.765 114.3) (width 0.254) (layer B.Cu) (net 24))
 (segment (start 124.11 107.95) (end 145.415 107.95) (width 0.254) (layer B.Cu) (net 24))
 (segment (start 106.68 120.65) (end 112.395 120.65) (width 1.016) (layer B.Cu) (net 3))
 (segment (start 152.4 144.145) (end 152.4 147.193) (width 1.016) (layer F.Cu) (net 3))
 (segment (start 156.21 140.335) (end 152.4 144.145) (width 1.016) (layer F.Cu) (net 3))
 (via (at 156.21 140.335) (size 0.889) (layers F.Cu B.Cu) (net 3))
 (segment (start 156.21 136.525) (end 156.21 140.335) (width 1.016) (layer B.Cu) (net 3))
 (segment (start 152.4 132.715) (end 156.21 136.525) (width 1.016) (layer B.Cu) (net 3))
 (segment (start 124.46 132.715) (end 152.4 132.715) (width 1.016) (layer B.Cu) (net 3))
 (segment (start 112.395 120.65) (end 124.46 132.715) (width 1.016) (layer B.Cu) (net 3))
 (segment (start 104.14 120.65) (end 106.68 120.65) (width 1.016) (layer B.Cu) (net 3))
 (segment (start 122.555 121.92) (end 122.555 120.65) (width 1.016) (layer B.Cu) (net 25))
 (segment (start 116.515 114.61) (end 116.515 113.665) (width 1.016) (layer B.Cu) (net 25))
 (segment (start 122.555 120.65) (end 116.515 114.61) (width 1.016) (layer B.Cu) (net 25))
 (segment (start 116.515 113.665) (end 116.515 111.045) (width 1.016) (layer F.Cu) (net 25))
 (segment (start 140.335 121.92) (end 140.335 120.65) (width 1.016) (layer B.Cu) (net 16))
 (segment (start 134.295 114.61) (end 134.295 113.665) (width 1.016) (layer B.Cu) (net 16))
 (segment (start 140.335 120.65) (end 134.295 114.61) (width 1.016) (layer B.Cu) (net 16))
 (segment (start 134.295 113.665) (end 134.295 111.045) (width 1.016) (layer F.Cu) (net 16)))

